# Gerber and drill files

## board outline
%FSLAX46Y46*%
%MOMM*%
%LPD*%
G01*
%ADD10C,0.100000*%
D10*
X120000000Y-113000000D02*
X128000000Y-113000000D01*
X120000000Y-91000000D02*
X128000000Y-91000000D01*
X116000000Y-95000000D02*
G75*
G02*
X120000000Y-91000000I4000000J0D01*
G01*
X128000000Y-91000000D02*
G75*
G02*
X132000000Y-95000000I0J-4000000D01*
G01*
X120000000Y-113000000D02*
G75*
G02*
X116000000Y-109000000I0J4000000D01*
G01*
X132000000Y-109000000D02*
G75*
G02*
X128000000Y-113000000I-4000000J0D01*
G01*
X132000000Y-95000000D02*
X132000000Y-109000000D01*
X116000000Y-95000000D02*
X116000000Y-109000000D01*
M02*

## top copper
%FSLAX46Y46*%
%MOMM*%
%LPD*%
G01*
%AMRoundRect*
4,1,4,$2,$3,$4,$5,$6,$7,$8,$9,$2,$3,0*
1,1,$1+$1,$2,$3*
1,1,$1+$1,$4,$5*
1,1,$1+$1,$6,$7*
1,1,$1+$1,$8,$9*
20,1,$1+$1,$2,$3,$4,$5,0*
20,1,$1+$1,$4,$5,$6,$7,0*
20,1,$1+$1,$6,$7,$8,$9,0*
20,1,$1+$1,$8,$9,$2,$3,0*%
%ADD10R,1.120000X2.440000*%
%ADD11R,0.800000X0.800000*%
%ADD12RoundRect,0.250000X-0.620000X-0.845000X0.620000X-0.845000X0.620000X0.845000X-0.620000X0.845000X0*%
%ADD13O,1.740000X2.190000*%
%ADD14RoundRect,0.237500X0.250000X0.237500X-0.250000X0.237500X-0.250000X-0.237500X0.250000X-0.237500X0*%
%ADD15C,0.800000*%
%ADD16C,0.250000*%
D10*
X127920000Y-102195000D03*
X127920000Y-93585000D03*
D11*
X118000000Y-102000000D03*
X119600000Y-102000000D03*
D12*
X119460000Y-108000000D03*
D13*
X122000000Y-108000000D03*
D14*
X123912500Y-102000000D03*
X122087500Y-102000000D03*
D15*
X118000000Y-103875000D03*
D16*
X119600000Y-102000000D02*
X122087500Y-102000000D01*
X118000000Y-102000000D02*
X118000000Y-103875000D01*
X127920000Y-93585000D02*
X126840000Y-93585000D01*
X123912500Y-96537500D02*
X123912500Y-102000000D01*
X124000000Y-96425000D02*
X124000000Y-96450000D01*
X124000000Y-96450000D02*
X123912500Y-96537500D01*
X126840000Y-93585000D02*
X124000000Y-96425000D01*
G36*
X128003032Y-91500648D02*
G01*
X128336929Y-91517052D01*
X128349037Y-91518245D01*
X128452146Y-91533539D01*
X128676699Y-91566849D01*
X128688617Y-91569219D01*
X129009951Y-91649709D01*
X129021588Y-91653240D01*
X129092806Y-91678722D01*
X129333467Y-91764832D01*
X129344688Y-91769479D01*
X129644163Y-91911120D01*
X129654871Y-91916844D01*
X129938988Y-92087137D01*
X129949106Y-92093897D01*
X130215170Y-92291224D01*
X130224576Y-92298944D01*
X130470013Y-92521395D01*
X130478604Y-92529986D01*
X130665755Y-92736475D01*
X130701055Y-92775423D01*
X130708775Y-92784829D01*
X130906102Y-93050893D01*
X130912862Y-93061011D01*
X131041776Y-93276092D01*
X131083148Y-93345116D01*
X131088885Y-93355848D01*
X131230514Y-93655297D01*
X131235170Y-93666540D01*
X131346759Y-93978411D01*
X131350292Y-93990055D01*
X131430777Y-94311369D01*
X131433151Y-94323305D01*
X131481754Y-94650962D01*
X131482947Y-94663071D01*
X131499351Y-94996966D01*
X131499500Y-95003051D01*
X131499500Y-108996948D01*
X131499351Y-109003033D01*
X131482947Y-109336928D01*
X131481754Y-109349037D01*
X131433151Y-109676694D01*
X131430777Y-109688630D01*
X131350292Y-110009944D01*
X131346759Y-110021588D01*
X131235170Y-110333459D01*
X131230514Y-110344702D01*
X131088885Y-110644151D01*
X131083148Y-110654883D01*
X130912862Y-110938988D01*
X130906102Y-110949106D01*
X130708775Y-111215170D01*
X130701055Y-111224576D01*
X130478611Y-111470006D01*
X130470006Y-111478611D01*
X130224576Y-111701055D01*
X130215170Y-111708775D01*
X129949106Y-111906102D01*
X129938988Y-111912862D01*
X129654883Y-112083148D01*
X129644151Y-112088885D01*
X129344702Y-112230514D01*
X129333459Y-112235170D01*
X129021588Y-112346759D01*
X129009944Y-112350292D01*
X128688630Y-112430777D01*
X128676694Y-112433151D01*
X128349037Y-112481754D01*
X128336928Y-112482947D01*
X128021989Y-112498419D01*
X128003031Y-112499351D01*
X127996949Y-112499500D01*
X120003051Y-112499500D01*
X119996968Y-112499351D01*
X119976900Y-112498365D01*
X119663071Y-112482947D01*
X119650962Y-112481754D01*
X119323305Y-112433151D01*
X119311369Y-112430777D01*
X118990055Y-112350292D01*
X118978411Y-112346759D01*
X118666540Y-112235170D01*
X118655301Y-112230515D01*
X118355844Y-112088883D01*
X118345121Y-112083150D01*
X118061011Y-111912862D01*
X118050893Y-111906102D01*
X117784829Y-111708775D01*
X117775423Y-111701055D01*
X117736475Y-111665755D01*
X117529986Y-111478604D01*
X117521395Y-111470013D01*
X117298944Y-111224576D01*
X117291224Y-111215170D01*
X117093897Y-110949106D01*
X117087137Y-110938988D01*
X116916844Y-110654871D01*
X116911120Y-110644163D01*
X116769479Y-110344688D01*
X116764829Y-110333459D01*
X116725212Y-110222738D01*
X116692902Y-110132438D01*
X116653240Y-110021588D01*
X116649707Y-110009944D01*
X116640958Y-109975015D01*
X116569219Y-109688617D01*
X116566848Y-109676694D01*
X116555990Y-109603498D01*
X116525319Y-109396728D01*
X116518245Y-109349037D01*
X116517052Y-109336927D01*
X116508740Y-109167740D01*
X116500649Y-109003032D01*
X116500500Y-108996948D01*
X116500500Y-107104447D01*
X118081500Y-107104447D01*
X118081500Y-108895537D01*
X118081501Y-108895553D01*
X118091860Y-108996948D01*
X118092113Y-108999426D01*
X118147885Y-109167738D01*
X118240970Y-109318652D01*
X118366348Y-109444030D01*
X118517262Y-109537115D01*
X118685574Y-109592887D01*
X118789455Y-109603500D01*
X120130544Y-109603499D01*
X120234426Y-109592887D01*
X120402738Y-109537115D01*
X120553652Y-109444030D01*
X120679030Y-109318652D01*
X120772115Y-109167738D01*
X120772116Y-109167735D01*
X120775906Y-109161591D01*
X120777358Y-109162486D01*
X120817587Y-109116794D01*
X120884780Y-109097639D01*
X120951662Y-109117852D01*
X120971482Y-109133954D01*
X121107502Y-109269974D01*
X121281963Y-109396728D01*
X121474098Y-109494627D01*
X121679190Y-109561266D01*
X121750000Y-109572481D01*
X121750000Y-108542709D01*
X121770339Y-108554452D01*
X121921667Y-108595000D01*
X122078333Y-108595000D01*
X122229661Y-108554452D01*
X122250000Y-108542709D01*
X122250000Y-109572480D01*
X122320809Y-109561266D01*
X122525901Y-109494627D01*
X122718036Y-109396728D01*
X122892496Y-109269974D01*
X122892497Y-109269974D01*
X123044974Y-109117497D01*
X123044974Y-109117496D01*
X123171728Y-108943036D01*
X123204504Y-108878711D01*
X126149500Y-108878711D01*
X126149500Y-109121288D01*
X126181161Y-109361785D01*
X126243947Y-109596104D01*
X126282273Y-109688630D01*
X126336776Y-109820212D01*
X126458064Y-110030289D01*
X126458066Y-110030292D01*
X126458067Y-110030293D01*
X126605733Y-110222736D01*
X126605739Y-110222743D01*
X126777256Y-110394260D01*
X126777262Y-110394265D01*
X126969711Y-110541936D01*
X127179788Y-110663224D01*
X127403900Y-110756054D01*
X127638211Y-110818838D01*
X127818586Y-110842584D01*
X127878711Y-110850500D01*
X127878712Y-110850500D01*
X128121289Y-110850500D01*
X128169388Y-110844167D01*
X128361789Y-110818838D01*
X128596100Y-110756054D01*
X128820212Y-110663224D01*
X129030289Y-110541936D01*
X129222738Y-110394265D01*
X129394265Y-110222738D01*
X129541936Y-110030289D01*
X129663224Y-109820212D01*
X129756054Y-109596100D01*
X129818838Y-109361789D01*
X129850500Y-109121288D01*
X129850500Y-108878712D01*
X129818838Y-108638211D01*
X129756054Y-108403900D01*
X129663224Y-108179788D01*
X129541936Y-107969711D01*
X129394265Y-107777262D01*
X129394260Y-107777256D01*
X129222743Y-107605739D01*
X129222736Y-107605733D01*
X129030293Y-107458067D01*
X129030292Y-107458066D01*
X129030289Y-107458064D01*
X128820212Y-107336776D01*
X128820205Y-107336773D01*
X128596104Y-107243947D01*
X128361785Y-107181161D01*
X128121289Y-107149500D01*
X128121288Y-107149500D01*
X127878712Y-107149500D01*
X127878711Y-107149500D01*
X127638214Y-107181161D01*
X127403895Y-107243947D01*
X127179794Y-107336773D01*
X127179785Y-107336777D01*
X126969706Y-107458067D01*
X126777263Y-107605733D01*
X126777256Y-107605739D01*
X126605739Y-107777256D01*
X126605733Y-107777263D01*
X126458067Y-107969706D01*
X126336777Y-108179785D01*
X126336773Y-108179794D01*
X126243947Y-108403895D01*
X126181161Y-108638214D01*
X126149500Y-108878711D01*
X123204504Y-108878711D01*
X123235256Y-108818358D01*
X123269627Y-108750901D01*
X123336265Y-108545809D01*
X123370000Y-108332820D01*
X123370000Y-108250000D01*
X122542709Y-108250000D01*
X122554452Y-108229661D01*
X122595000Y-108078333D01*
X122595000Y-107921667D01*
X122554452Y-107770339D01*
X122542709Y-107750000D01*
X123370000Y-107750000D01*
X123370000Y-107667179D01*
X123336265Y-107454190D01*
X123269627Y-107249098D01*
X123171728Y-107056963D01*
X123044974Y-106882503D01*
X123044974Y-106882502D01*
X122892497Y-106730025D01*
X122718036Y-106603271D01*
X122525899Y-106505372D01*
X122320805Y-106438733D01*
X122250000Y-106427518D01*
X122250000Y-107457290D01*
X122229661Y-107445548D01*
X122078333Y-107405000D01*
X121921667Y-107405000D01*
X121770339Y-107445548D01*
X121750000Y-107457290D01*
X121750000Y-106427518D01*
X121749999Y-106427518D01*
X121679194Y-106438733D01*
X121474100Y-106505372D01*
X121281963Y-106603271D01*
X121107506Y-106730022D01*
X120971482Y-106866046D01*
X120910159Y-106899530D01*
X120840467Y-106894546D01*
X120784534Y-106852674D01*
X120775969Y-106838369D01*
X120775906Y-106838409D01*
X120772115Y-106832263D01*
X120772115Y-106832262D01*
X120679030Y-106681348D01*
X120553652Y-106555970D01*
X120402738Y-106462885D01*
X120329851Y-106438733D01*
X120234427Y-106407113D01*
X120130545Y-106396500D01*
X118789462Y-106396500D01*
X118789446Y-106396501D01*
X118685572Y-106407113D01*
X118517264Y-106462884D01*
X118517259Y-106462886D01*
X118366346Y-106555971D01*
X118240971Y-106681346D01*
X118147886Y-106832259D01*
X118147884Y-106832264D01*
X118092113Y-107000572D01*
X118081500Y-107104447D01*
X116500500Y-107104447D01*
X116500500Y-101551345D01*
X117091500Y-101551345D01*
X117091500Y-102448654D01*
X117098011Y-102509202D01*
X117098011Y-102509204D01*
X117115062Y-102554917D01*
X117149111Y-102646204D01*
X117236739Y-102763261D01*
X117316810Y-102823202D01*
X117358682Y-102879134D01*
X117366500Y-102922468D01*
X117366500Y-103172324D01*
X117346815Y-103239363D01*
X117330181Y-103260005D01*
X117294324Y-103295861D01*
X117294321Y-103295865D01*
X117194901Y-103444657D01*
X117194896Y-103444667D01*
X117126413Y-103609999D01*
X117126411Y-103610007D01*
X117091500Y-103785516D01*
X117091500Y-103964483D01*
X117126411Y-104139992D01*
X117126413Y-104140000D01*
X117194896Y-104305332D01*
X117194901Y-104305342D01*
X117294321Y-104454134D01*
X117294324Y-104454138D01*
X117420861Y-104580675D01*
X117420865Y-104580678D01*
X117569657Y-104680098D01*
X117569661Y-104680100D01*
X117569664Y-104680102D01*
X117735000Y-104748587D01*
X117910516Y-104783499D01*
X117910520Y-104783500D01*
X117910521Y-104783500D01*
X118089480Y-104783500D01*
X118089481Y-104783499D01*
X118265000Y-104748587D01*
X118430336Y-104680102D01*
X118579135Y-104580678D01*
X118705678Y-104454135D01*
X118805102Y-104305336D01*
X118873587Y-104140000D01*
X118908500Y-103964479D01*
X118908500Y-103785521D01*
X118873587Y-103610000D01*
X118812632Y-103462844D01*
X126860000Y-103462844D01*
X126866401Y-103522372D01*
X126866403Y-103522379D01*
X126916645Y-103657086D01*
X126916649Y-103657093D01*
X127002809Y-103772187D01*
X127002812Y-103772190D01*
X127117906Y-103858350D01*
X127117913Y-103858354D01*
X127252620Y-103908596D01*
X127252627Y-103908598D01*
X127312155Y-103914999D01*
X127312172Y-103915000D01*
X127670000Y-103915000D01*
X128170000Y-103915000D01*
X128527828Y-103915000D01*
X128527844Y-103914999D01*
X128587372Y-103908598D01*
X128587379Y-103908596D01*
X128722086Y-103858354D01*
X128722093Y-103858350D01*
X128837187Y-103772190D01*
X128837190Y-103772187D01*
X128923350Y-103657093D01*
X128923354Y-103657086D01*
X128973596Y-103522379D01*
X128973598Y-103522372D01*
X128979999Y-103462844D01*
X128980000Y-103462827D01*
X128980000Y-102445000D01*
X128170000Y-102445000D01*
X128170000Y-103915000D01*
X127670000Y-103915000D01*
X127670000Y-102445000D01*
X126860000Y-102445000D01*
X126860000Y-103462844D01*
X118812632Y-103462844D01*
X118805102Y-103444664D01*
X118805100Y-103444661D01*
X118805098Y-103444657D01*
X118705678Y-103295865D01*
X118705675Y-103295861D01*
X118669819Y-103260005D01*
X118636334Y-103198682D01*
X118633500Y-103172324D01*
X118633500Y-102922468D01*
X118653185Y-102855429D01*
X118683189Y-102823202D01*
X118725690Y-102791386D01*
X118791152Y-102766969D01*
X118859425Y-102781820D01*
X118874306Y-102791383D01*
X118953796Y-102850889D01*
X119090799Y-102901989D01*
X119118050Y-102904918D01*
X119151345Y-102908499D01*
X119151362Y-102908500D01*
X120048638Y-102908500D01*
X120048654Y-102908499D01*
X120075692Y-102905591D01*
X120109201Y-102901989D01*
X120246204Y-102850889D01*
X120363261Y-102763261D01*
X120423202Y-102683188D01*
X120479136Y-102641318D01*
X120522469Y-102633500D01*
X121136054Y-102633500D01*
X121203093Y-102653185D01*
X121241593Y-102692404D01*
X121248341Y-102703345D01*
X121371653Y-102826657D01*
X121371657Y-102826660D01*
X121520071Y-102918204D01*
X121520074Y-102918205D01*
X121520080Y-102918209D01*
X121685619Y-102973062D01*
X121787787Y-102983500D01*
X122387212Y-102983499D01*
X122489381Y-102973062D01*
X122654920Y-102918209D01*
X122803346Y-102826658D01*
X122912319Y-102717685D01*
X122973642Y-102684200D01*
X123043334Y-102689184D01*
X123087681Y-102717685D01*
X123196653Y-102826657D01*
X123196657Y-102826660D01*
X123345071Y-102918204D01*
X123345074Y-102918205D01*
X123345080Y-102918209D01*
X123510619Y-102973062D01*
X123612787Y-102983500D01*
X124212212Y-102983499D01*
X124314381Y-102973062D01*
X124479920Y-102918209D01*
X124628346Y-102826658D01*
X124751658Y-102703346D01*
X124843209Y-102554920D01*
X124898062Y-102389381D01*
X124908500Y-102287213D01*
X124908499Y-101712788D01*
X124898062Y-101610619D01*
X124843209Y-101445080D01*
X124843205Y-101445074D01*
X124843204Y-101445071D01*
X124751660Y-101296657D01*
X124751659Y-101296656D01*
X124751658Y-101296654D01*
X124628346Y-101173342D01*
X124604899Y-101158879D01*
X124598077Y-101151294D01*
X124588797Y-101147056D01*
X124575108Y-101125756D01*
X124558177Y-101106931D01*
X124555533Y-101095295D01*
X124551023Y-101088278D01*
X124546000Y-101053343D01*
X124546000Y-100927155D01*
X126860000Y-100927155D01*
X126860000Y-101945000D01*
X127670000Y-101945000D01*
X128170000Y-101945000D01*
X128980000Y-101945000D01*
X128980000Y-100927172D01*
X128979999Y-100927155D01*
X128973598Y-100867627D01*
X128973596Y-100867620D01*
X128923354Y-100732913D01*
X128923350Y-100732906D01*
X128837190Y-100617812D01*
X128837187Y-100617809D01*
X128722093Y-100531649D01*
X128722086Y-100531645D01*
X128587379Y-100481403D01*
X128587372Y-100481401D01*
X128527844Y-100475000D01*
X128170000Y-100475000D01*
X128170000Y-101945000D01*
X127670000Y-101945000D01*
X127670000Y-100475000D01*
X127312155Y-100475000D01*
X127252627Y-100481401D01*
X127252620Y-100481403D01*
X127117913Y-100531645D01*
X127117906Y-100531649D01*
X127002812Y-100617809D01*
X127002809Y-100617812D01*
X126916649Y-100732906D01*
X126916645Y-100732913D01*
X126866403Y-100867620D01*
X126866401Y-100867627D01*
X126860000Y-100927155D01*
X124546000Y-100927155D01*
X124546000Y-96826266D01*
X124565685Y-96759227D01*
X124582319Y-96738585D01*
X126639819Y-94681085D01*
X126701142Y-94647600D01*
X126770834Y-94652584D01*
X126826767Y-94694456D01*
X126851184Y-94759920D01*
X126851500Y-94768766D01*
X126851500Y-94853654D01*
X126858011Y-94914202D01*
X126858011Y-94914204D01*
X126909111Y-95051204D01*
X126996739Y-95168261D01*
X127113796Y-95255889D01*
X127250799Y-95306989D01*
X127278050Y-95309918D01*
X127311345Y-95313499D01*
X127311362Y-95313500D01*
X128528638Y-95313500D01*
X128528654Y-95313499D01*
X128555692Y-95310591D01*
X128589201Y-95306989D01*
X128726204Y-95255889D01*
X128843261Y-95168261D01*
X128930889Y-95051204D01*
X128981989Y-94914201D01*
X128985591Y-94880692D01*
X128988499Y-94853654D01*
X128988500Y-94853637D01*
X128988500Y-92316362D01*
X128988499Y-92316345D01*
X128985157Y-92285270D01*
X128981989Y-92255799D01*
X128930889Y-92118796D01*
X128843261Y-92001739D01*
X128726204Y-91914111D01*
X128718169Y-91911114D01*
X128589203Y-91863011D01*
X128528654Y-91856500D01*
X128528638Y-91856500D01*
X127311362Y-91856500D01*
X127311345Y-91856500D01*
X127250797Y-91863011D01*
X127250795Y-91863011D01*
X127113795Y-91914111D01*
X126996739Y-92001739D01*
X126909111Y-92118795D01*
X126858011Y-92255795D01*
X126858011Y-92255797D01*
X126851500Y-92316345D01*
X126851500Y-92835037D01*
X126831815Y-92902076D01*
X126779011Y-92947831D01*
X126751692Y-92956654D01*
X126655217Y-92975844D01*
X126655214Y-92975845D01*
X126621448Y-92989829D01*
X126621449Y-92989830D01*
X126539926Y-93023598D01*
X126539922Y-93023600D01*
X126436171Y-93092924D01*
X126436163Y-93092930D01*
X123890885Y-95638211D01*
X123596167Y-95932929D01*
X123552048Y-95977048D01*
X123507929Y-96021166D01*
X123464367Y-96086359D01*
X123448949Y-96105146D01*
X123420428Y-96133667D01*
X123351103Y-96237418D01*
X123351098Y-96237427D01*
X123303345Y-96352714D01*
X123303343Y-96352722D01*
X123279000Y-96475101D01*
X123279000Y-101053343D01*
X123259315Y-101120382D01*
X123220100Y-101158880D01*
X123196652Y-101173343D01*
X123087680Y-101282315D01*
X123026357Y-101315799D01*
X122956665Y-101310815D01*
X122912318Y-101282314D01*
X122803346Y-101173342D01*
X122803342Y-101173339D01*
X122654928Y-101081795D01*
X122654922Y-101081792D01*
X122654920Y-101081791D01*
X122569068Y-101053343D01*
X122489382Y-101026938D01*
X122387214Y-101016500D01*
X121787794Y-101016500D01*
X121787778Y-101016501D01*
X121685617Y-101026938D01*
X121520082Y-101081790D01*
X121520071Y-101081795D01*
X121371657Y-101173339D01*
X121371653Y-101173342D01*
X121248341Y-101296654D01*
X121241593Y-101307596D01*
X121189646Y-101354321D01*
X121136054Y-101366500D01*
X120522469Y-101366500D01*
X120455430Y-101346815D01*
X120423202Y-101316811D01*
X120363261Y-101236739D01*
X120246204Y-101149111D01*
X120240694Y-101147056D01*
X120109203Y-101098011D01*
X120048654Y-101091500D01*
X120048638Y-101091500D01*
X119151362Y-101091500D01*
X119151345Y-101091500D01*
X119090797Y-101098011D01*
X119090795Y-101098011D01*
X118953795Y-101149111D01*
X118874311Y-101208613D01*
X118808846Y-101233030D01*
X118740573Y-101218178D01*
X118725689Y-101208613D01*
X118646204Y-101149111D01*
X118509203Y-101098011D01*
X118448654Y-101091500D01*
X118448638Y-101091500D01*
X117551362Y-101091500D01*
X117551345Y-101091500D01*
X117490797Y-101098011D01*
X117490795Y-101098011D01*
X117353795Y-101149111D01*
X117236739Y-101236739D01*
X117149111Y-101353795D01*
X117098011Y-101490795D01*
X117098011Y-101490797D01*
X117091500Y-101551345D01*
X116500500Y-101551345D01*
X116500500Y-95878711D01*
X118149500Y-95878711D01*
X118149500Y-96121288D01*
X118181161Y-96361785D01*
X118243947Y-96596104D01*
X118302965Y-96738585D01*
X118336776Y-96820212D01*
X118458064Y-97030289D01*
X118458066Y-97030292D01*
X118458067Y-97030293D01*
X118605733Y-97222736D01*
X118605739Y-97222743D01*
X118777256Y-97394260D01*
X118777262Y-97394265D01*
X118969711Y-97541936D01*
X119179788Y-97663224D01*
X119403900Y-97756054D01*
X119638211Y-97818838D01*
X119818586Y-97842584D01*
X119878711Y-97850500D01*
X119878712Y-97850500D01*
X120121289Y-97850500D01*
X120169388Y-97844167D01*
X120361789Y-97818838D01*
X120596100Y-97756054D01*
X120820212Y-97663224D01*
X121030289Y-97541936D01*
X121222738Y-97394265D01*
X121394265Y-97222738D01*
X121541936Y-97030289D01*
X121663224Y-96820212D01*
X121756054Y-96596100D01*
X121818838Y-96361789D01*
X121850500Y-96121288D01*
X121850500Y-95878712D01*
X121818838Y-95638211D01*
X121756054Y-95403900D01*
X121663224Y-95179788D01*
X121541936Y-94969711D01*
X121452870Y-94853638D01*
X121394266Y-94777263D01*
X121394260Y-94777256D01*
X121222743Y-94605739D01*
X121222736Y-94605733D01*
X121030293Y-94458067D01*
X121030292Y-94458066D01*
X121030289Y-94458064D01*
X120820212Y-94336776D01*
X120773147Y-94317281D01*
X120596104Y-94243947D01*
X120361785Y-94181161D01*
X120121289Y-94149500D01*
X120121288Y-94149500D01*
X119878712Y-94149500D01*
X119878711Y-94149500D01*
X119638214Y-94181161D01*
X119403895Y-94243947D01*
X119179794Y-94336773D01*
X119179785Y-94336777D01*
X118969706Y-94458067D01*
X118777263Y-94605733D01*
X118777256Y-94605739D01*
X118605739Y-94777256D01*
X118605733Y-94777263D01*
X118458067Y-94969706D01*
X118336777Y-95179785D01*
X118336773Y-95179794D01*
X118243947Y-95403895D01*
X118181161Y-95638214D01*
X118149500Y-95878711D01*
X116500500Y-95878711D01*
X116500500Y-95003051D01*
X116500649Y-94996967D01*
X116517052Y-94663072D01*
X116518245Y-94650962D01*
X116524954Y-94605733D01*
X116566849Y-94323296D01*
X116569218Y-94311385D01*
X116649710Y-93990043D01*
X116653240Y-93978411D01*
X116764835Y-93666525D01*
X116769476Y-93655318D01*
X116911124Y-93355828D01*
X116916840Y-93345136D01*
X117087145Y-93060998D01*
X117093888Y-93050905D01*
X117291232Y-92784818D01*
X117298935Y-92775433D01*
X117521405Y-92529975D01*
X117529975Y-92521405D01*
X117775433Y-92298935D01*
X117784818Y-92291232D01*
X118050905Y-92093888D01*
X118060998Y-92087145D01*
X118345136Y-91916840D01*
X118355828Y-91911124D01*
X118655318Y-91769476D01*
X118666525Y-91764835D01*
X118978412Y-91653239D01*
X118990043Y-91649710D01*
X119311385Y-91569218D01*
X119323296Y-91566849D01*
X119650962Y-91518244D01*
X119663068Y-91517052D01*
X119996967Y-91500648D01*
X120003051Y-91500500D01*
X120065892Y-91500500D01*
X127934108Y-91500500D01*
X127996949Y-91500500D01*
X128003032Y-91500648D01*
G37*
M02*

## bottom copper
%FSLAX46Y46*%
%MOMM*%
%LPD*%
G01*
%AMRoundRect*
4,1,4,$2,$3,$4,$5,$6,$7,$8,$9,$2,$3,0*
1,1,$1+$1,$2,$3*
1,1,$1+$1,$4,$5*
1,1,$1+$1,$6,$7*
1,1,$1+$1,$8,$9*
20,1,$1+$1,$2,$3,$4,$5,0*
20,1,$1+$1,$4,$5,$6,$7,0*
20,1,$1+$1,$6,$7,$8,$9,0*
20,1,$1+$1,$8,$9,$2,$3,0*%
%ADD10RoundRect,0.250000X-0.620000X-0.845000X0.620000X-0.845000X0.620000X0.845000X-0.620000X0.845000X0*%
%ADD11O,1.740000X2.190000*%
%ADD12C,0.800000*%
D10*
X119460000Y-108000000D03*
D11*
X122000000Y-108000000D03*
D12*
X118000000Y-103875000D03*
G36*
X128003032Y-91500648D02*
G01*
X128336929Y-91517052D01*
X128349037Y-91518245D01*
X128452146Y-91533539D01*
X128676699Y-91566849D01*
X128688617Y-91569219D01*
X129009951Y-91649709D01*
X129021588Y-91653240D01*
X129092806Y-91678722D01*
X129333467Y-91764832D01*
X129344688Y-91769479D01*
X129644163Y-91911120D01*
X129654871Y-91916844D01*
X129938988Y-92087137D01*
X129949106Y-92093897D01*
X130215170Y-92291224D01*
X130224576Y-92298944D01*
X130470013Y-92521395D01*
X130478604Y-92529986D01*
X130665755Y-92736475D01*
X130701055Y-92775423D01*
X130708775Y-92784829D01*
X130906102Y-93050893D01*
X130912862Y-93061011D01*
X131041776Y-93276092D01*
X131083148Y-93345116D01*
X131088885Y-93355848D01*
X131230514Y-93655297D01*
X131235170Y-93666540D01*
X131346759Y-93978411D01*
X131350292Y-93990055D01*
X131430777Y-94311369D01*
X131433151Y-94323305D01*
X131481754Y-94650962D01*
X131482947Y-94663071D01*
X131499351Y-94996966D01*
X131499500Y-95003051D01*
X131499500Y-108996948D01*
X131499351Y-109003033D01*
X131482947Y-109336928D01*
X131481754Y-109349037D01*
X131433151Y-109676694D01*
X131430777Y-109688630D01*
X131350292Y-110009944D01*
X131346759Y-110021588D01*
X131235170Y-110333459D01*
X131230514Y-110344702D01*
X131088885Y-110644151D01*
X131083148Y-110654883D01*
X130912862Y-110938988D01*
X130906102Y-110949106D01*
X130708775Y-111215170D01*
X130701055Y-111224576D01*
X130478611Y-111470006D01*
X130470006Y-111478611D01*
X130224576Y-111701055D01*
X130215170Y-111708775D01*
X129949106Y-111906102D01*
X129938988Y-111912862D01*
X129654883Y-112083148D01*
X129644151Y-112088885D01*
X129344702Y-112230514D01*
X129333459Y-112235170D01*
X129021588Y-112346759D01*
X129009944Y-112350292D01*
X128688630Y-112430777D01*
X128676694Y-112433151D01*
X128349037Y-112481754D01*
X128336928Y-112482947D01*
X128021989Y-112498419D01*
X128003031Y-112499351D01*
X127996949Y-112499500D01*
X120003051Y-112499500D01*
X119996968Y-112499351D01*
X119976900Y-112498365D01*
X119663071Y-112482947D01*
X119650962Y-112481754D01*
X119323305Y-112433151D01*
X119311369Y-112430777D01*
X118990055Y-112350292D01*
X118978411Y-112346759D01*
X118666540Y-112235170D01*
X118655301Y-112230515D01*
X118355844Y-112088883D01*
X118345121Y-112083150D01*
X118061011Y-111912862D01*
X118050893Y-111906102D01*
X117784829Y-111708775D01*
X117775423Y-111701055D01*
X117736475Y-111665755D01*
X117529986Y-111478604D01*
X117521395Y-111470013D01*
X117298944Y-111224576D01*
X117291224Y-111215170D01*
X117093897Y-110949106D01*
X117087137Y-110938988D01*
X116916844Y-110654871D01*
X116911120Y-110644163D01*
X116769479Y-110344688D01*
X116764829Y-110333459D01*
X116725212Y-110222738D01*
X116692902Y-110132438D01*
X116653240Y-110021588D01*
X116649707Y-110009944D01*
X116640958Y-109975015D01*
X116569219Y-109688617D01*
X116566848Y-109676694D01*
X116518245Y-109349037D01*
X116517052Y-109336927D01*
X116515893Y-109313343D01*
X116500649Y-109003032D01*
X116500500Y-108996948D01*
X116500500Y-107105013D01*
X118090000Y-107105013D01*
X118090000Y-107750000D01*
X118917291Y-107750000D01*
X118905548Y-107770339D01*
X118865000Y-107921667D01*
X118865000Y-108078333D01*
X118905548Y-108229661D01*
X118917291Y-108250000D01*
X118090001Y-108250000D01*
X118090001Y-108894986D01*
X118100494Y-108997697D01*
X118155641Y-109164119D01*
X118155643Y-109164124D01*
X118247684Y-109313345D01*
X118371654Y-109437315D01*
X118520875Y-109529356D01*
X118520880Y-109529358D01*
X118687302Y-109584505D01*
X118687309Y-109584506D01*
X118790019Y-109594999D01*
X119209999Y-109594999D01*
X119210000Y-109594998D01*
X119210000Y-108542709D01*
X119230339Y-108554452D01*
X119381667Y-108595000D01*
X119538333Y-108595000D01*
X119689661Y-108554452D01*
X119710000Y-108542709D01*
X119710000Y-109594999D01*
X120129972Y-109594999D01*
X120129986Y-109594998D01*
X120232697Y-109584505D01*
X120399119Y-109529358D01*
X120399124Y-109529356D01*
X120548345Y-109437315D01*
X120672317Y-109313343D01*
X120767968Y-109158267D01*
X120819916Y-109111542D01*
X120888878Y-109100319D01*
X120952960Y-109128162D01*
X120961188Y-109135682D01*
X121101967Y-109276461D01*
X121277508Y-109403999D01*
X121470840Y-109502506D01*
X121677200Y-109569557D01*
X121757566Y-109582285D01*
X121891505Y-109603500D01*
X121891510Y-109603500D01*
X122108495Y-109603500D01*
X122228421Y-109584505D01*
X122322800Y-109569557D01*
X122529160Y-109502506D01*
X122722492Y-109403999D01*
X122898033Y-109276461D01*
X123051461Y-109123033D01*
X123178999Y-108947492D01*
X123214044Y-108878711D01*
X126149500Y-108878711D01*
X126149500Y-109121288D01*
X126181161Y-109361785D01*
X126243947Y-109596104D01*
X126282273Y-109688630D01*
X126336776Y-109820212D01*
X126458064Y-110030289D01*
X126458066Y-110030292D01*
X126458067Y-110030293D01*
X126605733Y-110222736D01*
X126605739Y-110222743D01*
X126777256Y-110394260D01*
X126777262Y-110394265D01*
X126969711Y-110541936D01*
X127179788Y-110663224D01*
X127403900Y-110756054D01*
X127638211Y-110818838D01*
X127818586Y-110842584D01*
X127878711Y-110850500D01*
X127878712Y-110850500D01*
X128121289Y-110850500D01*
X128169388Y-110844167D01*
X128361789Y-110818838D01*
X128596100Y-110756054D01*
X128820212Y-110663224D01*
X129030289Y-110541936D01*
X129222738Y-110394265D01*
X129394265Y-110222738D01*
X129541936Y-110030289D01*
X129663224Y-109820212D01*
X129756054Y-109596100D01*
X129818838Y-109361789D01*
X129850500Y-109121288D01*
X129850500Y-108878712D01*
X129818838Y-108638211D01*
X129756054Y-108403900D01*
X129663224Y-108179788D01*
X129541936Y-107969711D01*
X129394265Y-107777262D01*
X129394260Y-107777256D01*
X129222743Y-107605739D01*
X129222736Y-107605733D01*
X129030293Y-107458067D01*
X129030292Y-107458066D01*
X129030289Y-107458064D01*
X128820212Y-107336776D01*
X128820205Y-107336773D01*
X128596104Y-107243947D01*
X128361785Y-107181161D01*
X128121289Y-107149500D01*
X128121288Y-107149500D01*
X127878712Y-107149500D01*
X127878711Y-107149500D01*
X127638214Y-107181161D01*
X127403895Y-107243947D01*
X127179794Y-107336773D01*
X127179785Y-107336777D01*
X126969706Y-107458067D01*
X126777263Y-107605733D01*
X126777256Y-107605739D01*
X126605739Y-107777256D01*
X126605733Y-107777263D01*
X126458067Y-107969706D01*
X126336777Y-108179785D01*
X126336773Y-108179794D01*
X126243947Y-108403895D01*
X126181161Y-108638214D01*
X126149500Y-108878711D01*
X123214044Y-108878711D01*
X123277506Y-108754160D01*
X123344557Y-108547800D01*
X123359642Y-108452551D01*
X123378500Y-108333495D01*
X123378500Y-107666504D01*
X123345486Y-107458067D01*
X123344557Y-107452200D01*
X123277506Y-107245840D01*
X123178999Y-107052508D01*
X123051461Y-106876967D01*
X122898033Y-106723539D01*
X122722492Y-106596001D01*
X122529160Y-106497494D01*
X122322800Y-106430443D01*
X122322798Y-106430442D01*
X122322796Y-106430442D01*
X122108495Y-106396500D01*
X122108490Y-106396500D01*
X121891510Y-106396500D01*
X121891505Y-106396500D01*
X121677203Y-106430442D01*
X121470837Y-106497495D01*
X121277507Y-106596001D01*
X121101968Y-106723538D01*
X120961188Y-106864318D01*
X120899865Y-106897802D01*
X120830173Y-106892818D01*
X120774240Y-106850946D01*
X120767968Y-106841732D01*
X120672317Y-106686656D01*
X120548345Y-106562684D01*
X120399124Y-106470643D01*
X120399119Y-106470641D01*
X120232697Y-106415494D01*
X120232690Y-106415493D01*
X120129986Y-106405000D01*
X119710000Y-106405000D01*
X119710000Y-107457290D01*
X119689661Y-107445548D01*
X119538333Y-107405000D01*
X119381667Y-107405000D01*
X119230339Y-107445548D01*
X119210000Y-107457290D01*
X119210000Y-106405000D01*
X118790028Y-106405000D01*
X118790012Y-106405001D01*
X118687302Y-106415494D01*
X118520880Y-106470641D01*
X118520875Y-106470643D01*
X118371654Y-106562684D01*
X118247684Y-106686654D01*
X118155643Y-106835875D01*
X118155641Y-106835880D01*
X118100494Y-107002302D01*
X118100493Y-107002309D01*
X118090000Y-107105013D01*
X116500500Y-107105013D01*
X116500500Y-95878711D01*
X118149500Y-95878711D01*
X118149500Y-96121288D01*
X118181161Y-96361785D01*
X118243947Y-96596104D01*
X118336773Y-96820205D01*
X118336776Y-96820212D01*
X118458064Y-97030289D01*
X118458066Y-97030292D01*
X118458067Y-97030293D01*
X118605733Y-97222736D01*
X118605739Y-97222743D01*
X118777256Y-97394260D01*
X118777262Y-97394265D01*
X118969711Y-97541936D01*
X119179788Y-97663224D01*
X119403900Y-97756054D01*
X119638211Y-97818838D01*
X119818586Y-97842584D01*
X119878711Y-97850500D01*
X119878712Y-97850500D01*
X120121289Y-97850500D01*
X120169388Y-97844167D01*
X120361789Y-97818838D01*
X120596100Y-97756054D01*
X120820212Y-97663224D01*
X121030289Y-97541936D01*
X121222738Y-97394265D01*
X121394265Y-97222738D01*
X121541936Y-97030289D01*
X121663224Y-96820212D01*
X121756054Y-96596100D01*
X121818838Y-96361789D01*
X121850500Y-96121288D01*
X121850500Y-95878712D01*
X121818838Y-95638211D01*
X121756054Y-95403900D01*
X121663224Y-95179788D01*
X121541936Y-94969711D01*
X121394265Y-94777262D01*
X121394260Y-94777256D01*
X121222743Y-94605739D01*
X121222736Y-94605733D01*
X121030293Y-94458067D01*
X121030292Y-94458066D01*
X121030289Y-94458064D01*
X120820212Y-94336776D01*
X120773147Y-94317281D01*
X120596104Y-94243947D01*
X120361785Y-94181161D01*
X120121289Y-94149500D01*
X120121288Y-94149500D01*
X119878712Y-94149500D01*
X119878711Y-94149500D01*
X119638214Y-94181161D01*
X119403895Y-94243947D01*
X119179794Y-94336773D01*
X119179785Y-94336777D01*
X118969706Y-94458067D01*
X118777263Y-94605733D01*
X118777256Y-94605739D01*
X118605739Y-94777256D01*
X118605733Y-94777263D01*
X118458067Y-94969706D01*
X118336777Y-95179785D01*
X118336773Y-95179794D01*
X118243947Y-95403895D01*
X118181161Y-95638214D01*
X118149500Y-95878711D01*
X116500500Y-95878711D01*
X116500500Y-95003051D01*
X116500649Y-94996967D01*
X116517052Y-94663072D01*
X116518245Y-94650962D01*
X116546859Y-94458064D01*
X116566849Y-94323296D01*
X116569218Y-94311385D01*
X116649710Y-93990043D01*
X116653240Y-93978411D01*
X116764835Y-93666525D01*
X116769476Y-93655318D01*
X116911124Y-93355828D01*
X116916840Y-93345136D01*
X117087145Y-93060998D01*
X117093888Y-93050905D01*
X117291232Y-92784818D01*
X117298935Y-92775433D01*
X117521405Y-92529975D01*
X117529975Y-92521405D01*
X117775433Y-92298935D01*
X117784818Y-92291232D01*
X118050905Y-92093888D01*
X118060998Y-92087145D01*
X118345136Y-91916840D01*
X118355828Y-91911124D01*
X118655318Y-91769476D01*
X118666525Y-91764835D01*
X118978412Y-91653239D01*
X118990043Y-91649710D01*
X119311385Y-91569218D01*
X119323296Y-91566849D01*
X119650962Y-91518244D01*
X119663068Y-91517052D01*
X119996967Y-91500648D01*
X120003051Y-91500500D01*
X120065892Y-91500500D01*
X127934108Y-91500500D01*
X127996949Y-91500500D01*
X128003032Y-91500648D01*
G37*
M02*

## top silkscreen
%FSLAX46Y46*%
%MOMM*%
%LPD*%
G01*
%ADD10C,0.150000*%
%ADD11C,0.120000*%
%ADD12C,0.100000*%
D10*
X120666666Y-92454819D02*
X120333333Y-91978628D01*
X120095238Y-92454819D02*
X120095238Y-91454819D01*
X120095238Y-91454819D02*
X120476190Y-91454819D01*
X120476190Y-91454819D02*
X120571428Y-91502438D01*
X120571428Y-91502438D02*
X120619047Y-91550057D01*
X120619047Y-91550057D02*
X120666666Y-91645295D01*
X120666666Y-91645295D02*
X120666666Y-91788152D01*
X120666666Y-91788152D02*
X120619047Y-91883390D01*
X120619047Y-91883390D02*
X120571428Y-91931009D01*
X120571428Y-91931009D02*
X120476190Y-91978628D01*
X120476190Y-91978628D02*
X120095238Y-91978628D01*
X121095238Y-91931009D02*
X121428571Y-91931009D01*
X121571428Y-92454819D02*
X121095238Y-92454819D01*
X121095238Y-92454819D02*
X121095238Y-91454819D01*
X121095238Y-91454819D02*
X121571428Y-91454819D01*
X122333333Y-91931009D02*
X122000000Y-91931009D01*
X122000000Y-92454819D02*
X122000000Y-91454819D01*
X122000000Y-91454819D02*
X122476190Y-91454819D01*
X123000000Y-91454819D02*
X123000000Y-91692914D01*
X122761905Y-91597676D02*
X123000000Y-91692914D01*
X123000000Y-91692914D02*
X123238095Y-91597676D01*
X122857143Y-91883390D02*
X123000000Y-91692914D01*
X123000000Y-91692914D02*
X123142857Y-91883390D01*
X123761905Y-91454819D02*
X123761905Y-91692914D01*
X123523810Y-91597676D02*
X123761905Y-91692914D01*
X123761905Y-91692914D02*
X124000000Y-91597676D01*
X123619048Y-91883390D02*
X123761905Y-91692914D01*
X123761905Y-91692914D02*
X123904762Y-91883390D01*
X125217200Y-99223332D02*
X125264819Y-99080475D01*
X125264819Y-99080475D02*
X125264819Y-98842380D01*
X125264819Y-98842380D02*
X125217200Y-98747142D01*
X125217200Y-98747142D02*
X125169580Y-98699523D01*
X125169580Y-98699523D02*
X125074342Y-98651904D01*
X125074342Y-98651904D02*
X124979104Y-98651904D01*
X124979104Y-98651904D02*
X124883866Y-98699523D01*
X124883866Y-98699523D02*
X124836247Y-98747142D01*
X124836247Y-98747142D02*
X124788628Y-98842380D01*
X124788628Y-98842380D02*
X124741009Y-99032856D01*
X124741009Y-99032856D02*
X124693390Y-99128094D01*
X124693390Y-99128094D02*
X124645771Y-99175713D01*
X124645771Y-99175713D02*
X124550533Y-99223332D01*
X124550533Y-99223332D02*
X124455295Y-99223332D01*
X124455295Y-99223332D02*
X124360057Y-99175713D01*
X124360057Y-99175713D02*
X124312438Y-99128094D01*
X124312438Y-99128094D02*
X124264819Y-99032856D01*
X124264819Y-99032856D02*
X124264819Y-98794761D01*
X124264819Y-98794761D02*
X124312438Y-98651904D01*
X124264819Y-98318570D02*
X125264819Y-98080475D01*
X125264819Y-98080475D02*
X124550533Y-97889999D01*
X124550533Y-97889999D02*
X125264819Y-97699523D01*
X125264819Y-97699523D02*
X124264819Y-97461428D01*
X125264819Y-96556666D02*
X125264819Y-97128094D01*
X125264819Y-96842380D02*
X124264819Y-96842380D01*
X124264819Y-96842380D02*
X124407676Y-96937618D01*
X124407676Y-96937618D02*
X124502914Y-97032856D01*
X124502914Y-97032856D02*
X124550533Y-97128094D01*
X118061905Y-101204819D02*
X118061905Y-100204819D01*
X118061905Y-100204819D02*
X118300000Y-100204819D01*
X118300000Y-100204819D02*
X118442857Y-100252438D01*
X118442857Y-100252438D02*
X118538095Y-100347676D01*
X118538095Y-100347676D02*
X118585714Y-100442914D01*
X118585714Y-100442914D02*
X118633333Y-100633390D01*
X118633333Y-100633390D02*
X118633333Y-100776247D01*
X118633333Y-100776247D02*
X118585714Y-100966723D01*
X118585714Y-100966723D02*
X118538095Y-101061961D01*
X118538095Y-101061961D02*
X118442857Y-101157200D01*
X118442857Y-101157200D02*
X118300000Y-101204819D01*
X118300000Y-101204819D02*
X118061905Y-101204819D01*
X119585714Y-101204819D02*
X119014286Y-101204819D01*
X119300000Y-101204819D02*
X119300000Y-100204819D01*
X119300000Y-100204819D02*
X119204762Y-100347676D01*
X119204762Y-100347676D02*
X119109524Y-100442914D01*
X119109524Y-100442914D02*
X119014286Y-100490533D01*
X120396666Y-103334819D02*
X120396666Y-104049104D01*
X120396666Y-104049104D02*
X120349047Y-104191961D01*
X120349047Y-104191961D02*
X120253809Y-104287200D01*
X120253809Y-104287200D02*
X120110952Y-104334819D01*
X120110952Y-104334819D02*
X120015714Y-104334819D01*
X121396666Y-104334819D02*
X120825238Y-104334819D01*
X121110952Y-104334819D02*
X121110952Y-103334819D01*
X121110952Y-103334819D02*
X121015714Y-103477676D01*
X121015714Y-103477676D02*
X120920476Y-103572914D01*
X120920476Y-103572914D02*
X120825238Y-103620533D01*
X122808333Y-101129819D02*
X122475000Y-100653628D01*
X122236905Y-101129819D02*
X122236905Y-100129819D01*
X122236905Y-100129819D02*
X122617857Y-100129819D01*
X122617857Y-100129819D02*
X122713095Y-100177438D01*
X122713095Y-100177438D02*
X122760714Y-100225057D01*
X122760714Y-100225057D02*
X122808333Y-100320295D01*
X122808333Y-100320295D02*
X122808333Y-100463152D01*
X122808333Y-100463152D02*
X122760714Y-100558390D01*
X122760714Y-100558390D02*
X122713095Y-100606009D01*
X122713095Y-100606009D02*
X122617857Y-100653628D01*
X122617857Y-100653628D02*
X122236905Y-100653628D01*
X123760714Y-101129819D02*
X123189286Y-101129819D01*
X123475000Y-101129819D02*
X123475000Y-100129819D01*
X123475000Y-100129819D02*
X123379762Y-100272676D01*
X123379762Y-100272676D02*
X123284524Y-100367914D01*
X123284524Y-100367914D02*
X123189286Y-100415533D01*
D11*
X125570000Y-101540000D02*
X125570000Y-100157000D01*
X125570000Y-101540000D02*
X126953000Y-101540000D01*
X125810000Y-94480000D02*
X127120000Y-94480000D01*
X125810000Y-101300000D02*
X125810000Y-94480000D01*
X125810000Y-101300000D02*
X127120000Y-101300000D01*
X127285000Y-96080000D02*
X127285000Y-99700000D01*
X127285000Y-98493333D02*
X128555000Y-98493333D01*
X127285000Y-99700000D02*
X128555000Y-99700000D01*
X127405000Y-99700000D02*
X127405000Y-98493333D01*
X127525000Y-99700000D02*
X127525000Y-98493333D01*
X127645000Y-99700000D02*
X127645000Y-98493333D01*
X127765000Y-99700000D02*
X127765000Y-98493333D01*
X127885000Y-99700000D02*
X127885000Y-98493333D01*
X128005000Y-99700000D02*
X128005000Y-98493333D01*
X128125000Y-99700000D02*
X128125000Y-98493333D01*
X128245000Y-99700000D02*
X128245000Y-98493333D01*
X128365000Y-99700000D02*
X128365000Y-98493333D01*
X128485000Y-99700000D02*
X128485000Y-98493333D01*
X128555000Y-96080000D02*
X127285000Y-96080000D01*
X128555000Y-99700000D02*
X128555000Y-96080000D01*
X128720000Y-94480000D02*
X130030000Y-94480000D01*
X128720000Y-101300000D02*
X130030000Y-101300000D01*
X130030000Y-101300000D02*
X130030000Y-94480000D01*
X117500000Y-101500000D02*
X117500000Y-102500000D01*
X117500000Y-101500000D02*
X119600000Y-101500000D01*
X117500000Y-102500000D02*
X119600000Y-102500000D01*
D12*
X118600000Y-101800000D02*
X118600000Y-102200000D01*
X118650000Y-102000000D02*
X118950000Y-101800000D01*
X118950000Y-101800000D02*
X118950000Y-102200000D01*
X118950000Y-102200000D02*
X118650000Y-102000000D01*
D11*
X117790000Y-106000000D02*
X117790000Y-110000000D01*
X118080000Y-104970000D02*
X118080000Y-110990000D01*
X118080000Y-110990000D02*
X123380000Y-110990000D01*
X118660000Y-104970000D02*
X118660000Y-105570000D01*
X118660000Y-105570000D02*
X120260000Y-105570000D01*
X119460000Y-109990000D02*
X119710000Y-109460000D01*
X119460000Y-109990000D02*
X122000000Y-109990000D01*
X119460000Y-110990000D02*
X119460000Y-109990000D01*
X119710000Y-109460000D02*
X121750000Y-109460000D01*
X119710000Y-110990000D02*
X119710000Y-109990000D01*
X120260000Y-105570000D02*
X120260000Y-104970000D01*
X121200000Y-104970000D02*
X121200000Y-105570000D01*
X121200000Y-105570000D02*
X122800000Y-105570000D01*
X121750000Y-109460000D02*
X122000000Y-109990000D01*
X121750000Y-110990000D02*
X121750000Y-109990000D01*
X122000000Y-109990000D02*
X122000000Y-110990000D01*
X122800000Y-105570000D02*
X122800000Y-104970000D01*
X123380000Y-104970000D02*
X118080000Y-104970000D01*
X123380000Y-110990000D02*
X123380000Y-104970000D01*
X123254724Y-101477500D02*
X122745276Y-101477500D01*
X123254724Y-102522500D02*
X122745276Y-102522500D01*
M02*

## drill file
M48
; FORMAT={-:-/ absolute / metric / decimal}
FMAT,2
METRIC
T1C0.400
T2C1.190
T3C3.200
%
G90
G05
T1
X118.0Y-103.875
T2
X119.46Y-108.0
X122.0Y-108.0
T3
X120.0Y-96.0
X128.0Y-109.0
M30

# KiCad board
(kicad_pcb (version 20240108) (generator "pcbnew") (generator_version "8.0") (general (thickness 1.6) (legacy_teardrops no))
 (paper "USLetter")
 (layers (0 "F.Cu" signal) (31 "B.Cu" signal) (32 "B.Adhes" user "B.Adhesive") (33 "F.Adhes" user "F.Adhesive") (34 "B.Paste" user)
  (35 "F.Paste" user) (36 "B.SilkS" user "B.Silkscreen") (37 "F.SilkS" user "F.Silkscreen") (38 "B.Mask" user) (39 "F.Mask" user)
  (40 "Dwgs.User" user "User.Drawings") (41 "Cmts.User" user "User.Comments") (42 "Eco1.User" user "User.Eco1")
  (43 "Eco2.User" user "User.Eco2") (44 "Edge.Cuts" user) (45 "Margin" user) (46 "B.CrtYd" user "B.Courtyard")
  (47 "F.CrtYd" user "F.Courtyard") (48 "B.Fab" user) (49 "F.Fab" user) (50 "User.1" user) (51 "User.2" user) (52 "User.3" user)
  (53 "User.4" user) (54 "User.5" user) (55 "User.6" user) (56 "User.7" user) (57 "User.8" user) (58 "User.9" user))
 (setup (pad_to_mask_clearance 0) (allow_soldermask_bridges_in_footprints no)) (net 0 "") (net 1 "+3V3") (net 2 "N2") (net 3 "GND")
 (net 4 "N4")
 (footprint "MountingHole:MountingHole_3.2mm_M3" (layer "F.Cu") (at 128 109)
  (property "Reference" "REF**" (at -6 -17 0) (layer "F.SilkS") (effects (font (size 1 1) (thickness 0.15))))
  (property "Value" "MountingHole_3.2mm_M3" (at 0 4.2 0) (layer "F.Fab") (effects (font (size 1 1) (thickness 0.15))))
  (pad "" np_thru_hole circle (at 0 0) (size 3.2 3.2) (drill 3.2) (layers "*.Cu" "*.Mask")))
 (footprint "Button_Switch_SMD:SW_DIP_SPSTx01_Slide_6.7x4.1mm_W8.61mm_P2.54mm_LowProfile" (layer "F.Cu") (at 127.92 97.89 90)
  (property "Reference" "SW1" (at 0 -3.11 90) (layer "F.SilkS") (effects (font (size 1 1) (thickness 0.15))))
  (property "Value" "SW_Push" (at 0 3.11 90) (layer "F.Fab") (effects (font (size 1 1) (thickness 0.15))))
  (fp_line (start -3.65 -2.35) (end -2.267 -2.35) (stroke (width 0.12) (type solid)) (layer "F.SilkS"))
  (fp_line (start -3.65 -2.35) (end -3.65 -0.967) (stroke (width 0.12) (type solid)) (layer "F.SilkS"))
  (fp_line (start 3.41 -2.11) (end 3.41 -0.8) (stroke (width 0.12) (type solid)) (layer "F.SilkS"))
  (fp_line (start -3.41 -2.11) (end 3.41 -2.11) (stroke (width 0.12) (type solid)) (layer "F.SilkS"))
  (fp_line (start -3.41 -2.11) (end -3.41 -0.8) (stroke (width 0.12) (type solid)) (layer "F.SilkS"))
  (fp_line (start 1.81 -0.635) (end -1.81 -0.635) (stroke (width 0.12) (type solid)) (layer "F.SilkS"))
  (fp_line (start -0.603333 -0.635) (end -0.603333 0.635) (stroke (width 0.12) (type solid)) (layer "F.SilkS"))
  (fp_line (start -1.81 -0.635) (end -1.81 0.635) (stroke (width 0.12) (type solid)) (layer "F.SilkS"))
  (fp_line (start -1.81 -0.515) (end -0.603333 -0.515) (stroke (width 0.12) (type solid)) (layer "F.SilkS"))
  (fp_line (start -1.81 -0.395) (end -0.603333 -0.395) (stroke (width 0.12) (type solid)) (layer "F.SilkS"))
  (fp_line (start -1.81 -0.275) (end -0.603333 -0.275) (stroke (width 0.12) (type solid)) (layer "F.SilkS"))
  (fp_line (start -1.81 -0.155) (end -0.603333 -0.155) (stroke (width 0.12) (type solid)) (layer "F.SilkS"))
  (fp_line (start -1.81 -0.035) (end -0.603333 -0.035) (stroke (width 0.12) (type solid)) (layer "F.SilkS"))
  (fp_line (start -1.81 0.085) (end -0.603333 0.085) (stroke (width 0.12) (type solid)) (layer "F.SilkS"))
  (fp_line (start -1.81 0.205) (end -0.603333 0.205) (stroke (width 0.12) (type solid)) (layer "F.SilkS"))
  (fp_line (start -1.81 0.325) (end -0.603333 0.325) (stroke (width 0.12) (type solid)) (layer "F.SilkS"))
  (fp_line (start -1.81 0.445) (end -0.603333 0.445) (stroke (width 0.12) (type solid)) (layer "F.SilkS"))
  (fp_line (start -1.81 0.565) (end -0.603333 0.565) (stroke (width 0.12) (type solid)) (layer "F.SilkS"))
  (fp_line (start 1.81 0.635) (end 1.81 -0.635) (stroke (width 0.12) (type solid)) (layer "F.SilkS"))
  (fp_line (start -1.81 0.635) (end 1.81 0.635) (stroke (width 0.12) (type solid)) (layer "F.SilkS"))
  (fp_line (start 3.41 0.8) (end 3.41 2.11) (stroke (width 0.12) (type solid)) (layer "F.SilkS"))
  (fp_line (start -3.41 0.8) (end -3.41 2.11) (stroke (width 0.12) (type solid)) (layer "F.SilkS"))
  (fp_line (start -3.41 2.11) (end 3.41 2.11) (stroke (width 0.12) (type solid)) (layer "F.SilkS"))
  (pad "1" smd rect (at -4.305 0 90) (size 2.44 1.12) (layers "F.Cu" "F.Paste" "F.Mask") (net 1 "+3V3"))
  (pad "2" smd rect (at 4.305 0 90) (size 2.44 1.12) (layers "F.Cu" "F.Paste" "F.Mask") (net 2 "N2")))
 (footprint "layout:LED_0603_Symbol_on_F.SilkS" (layer "F.Cu") (at 118.8 102)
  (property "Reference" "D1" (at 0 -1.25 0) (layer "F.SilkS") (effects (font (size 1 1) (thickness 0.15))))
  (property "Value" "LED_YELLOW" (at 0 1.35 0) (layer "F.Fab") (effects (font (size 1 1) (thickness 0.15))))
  (fp_line (start -1.3 -0.5) (end -1.3 0.5) (stroke (width 0.12) (type solid)) (layer "F.SilkS"))
  (fp_line (start -1.3 -0.5) (end 0.8 -0.5) (stroke (width 0.12) (type solid)) (layer "F.SilkS"))
  (fp_line (start -1.3 0.5) (end 0.8 0.5) (stroke (width 0.12) (type solid)) (layer "F.SilkS"))
  (fp_line (start -0.2 -0.2) (end -0.2 0.2) (stroke (width 0.1) (type solid)) (layer "F.SilkS"))
  (fp_line (start -0.15 0) (end 0.15 -0.2) (stroke (width 0.1) (type solid)) (layer "F.SilkS"))
  (fp_line (start 0.15 -0.2) (end 0.15 0.2) (stroke (width 0.1) (type solid)) (layer "F.SilkS"))
  (fp_line (start 0.15 0.2) (end -0.15 0) (stroke (width 0.1) (type solid)) (layer "F.SilkS"))
  (pad "1" smd rect (at -0.8 0 180) (size 0.8 0.8) (layers "F.Cu" "F.Paste" "F.Mask") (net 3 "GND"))
  (pad "2" smd rect (at 0.8 0 180) (size 0.8 0.8) (layers "F.Cu" "F.Paste" "F.Mask") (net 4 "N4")))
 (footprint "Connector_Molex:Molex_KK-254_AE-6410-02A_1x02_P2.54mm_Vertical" (layer "F.Cu") (at 119.46 108)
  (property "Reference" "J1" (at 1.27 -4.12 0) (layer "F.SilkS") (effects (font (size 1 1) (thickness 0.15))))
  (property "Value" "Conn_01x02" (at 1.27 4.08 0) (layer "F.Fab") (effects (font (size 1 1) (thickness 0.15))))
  (fp_line (start -1.67 -2) (end -1.67 2) (stroke (width 0.12) (type solid)) (layer "F.SilkS"))
  (fp_line (start -1.38 -3.03) (end -1.38 2.99) (stroke (width 0.12) (type solid)) (layer "F.SilkS"))
  (fp_line (start -1.38 2.99) (end 3.92 2.99) (stroke (width 0.12) (type solid)) (layer "F.SilkS"))
  (fp_line (start -0.8 -3.03) (end -0.8 -2.43) (stroke (width 0.12) (type solid)) (layer "F.SilkS"))
  (fp_line (start -0.8 -2.43) (end 0.8 -2.43) (stroke (width 0.12) (type solid)) (layer "F.SilkS"))
  (fp_line (start 0 1.99) (end 0.25 1.46) (stroke (width 0.12) (type solid)) (layer "F.SilkS"))
  (fp_line (start 0 1.99) (end 2.54 1.99) (stroke (width 0.12) (type solid)) (layer "F.SilkS"))
  (fp_line (start 0 2.99) (end 0 1.99) (stroke (width 0.12) (type solid)) (layer "F.SilkS"))
  (fp_line (start 0.25 1.46) (end 2.29 1.46) (stroke (width 0.12) (type solid)) (layer "F.SilkS"))
  (fp_line (start 0.25 2.99) (end 0.25 1.99) (stroke (width 0.12) (type solid)) (layer "F.SilkS"))
  (fp_line (start 0.8 -2.43) (end 0.8 -3.03) (stroke (width 0.12) (type solid)) (layer "F.SilkS"))
  (fp_line (start 1.74 -3.03) (end 1.74 -2.43) (stroke (width 0.12) (type solid)) (layer "F.SilkS"))
  (fp_line (start 1.74 -2.43) (end 3.34 -2.43) (stroke (width 0.12) (type solid)) (layer "F.SilkS"))
  (fp_line (start 2.29 1.46) (end 2.54 1.99) (stroke (width 0.12) (type solid)) (layer "F.SilkS"))
  (fp_line (start 2.29 2.99) (end 2.29 1.99) (stroke (width 0.12) (type solid)) (layer "F.SilkS"))
  (fp_line (start 2.54 1.99) (end 2.54 2.99) (stroke (width 0.12) (type solid)) (layer "F.SilkS"))
  (fp_line (start 3.34 -2.43) (end 3.34 -3.03) (stroke (width 0.12) (type solid)) (layer "F.SilkS"))
  (fp_line (start 3.92 -3.03) (end -1.38 -3.03) (stroke (width 0.12) (type solid)) (layer "F.SilkS"))
  (fp_line (start 3.92 2.99) (end 3.92 -3.03) (stroke (width 0.12) (type solid)) (layer "F.SilkS"))
  (pad "1" thru_hole roundrect (at 0 0) (size 1.74 2.19) (drill 1.19) (layers "*.Cu" "*.Mask") (remove_unused_layers no)
   (roundrect_rratio 0.143678) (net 3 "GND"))
  (pad "2" thru_hole oval (at 2.54 0) (size 1.74 2.19) (drill 1.19) (layers "*.Cu" "*.Mask") (remove_unused_layers no) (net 1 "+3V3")))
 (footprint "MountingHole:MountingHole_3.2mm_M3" (layer "F.Cu") (at 120 96)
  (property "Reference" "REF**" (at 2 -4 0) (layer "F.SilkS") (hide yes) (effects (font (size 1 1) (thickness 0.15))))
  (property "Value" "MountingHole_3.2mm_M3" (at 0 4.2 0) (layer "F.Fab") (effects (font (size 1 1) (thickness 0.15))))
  (pad "" np_thru_hole circle (at 0 0) (size 3.2 3.2) (drill 3.2) (layers "*.Cu" "*.Mask")))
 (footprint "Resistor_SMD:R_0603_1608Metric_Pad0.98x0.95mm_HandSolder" (layer "F.Cu") (at 123 102 180)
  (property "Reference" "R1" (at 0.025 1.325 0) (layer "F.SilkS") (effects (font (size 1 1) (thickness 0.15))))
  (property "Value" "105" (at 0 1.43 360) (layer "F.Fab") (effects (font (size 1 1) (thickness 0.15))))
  (fp_line (start -0.254724 0.5225) (end 0.254724 0.5225) (stroke (width 0.12) (type solid)) (layer "F.SilkS"))
  (fp_line (start -0.254724 -0.5225) (end 0.254724 -0.5225) (stroke (width 0.12) (type solid)) (layer "F.SilkS"))
  (pad "1" smd roundrect (at -0.9125 0 180) (size 0.975 0.95) (layers "F.Cu" "F.Paste" "F.Mask") (roundrect_rratio 0.25) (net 2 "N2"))
  (pad "2" smd roundrect (at 0.9125 0 180) (size 0.975 0.95) (layers "F.Cu" "F.Paste" "F.Mask") (roundrect_rratio 0.25) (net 4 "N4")))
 (gr_line (start 120 113) (end 128 113) (stroke (width 0.1) (type default)) (layer "Edge.Cuts"))
 (gr_line (start 120 91) (end 128 91) (stroke (width 0.1) (type default)) (layer "Edge.Cuts"))
 (gr_arc (start 116 95) (mid 117.171573 92.171573) (end 120 91) (stroke (width 0.1) (type default)) (layer "Edge.Cuts"))
 (gr_arc (start 128 91) (mid 130.828427 92.171573) (end 132 95) (stroke (width 0.1) (type default)) (layer "Edge.Cuts"))
 (gr_arc (start 120 113) (mid 117.171573 111.828427) (end 116 109) (stroke (width 0.1) (type default)) (layer "Edge.Cuts"))
 (gr_arc (start 132 109) (mid 130.828427 111.828427) (end 128 113) (stroke (width 0.1) (type default)) (layer "Edge.Cuts"))
 (gr_line (start 132 95) (end 132 109) (stroke (width 0.1) (type default)) (layer "Edge.Cuts"))
 (gr_line (start 116 95) (end 116 109) (stroke (width 0.1) (type default)) (layer "Edge.Cuts"))
 (segment (start 119.6 102) (end 122.0875 102) (width 0.25) (layer "F.Cu") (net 4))
 (segment (start 118 102) (end 118 103.875) (width 0.25) (layer "F.Cu") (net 3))
 (via (at 118 103.875) (size 0.8) (drill 0.4) (layers "F.Cu" "B.Cu") (free yes) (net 3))
 (segment (start 127.92 93.585) (end 126.84 93.585) (width 0.25) (layer "F.Cu") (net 2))
 (segment (start 123.9125 96.5375) (end 123.9125 102) (width 0.25) (layer "F.Cu") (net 2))
 (segment (start 124 96.425) (end 124 96.45) (width 0.25) (layer "F.Cu") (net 2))
 (segment (start 124 96.45) (end 123.9125 96.5375) (width 0.25) (layer "F.Cu") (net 2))
 (segment (start 126.84 93.585) (end 124 96.425) (width 0.25) (layer "F.Cu") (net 2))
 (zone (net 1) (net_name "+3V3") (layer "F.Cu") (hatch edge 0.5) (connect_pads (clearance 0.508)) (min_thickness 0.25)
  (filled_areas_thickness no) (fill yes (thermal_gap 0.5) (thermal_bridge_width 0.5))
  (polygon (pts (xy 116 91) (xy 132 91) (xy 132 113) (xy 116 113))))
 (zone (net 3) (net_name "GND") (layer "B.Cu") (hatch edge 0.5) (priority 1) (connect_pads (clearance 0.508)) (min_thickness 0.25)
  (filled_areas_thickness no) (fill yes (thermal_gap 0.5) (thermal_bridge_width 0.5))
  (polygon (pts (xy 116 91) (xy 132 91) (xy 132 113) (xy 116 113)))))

